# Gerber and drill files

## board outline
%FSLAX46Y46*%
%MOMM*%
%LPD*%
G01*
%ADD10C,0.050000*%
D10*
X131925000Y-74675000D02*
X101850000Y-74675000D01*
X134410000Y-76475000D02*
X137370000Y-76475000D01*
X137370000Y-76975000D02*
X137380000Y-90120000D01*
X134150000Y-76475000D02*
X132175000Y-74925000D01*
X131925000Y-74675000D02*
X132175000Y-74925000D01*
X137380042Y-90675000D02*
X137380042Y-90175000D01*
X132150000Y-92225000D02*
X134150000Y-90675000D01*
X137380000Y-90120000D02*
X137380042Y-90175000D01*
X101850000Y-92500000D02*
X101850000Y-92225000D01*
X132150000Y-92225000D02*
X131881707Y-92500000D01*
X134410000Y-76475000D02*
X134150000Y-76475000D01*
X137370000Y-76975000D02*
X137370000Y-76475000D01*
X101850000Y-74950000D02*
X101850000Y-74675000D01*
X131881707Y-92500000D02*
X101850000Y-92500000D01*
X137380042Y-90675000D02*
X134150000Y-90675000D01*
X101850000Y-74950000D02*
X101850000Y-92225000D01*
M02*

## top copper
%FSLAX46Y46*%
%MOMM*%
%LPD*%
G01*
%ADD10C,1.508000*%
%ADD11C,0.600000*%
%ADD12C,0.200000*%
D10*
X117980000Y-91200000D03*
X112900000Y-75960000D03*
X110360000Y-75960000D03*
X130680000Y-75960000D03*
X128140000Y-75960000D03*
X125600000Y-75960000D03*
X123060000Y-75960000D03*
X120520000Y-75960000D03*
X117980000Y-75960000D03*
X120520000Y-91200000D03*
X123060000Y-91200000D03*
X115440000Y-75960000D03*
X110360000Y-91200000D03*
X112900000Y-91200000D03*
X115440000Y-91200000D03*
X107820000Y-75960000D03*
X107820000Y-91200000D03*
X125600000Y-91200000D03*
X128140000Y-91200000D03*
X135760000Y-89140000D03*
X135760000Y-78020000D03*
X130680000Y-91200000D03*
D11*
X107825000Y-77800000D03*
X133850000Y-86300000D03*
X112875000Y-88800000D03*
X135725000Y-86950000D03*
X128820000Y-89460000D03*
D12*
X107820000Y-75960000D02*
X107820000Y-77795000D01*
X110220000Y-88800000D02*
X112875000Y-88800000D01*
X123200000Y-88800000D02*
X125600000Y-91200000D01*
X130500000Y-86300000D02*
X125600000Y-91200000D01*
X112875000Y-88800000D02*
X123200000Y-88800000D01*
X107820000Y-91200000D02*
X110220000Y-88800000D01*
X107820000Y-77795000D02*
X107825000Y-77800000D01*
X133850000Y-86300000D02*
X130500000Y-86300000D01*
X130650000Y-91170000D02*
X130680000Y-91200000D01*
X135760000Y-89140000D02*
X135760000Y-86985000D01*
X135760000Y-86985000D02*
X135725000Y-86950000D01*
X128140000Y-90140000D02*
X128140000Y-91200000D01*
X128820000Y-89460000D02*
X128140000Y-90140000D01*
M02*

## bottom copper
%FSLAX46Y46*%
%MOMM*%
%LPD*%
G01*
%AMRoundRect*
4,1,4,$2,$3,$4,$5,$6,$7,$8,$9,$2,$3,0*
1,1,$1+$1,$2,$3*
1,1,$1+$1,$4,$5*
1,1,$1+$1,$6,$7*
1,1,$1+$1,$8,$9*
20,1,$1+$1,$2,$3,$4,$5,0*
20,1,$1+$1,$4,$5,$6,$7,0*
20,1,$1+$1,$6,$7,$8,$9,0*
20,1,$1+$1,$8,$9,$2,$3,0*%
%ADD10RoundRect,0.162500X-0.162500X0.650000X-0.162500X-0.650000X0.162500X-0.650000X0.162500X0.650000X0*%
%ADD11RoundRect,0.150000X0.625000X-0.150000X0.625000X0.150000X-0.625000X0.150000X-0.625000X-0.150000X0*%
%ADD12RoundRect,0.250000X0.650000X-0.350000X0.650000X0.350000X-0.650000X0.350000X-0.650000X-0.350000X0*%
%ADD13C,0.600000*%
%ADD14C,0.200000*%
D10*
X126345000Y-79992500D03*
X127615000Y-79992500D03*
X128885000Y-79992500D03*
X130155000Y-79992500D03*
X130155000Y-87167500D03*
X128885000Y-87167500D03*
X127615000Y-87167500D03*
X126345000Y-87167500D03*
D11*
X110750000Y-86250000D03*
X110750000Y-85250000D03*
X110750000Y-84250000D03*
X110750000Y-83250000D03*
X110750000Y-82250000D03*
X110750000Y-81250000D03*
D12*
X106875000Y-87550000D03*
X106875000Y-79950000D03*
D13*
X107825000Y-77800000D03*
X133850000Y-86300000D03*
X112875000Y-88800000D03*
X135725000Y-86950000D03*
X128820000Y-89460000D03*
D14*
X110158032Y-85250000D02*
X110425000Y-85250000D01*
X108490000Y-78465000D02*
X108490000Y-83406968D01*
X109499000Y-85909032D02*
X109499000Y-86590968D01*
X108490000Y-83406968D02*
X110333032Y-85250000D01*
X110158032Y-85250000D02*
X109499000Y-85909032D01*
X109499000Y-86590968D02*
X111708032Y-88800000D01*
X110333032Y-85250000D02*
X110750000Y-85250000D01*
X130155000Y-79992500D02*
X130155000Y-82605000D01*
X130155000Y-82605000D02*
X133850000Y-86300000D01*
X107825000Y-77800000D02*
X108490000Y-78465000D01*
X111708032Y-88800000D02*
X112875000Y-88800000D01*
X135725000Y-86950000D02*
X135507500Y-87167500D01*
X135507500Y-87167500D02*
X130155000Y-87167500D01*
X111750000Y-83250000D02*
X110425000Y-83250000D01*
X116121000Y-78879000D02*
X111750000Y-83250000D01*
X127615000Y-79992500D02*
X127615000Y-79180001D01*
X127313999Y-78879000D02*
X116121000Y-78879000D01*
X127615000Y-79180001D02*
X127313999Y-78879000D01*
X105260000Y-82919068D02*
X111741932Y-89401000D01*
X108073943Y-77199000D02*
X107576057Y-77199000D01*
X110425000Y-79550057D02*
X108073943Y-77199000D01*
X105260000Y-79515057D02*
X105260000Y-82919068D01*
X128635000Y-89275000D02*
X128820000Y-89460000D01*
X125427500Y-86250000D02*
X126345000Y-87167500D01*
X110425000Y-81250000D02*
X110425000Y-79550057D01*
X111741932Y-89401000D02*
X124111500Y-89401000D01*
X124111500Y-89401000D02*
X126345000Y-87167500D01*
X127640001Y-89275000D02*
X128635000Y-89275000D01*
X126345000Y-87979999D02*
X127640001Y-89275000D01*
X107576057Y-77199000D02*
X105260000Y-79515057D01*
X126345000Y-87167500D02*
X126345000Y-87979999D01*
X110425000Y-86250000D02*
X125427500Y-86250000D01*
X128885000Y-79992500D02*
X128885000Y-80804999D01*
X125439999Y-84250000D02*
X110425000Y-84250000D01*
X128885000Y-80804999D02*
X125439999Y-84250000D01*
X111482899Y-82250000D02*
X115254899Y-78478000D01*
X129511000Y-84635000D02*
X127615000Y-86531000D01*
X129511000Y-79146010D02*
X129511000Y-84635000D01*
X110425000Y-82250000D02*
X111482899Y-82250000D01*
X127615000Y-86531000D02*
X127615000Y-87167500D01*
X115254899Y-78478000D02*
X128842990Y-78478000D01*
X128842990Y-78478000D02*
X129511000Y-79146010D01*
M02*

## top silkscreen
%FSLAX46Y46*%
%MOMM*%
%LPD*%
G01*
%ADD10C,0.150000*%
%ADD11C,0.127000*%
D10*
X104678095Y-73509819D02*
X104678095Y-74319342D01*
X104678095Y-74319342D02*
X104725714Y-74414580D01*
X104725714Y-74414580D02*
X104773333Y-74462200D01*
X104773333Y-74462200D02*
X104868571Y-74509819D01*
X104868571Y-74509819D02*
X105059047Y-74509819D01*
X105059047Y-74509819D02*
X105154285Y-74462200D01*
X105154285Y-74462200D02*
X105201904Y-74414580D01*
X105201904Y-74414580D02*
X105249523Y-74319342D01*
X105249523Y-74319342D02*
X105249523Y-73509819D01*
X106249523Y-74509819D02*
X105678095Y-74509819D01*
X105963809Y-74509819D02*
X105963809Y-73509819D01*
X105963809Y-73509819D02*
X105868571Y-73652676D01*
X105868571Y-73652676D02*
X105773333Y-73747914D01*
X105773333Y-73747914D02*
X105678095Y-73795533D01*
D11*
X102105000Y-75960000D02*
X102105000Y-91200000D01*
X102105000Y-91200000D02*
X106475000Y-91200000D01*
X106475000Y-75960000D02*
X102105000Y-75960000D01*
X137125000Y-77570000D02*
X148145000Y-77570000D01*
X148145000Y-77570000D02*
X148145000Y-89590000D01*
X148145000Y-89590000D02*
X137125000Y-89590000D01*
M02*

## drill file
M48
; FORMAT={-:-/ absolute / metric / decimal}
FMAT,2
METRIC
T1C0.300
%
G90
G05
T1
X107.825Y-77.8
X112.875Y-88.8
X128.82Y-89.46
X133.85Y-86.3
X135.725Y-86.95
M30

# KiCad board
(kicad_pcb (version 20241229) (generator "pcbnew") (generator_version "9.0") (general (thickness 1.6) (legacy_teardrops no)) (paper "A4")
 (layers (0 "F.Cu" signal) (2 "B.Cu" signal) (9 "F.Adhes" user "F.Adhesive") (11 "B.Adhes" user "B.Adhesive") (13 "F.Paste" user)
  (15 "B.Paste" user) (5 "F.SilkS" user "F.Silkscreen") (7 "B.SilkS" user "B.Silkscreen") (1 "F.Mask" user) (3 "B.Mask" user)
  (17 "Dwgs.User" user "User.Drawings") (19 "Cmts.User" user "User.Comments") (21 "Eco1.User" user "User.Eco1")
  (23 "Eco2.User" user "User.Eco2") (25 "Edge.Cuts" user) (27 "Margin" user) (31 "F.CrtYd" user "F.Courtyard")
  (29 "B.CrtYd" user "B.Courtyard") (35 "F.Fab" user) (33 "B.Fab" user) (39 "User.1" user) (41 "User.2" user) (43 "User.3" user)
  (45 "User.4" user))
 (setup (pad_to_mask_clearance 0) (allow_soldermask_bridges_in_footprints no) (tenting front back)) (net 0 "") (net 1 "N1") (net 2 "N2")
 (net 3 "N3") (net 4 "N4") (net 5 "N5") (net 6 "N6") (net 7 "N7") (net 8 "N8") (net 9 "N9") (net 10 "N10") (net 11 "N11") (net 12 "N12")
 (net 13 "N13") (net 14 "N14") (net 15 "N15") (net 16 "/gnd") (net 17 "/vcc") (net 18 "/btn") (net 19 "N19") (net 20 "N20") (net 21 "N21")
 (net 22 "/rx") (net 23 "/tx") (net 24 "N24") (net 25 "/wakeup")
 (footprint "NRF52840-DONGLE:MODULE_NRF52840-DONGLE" (layer "F.Cu") (at 125.125 83.58)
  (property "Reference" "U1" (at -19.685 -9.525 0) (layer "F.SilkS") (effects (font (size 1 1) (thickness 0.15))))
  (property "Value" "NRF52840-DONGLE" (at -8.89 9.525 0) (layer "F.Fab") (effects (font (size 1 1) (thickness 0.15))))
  (fp_line (start -23.02 -7.62) (end -23.02 7.62) (stroke (width 0.127) (type solid)) (layer "F.SilkS"))
  (fp_line (start -23.02 7.62) (end -18.65 7.62) (stroke (width 0.127) (type solid)) (layer "F.SilkS"))
  (fp_line (start -18.65 -7.62) (end -23.02 -7.62) (stroke (width 0.127) (type solid)) (layer "F.SilkS"))
  (fp_line (start 12 -6.01) (end 23.02 -6.01) (stroke (width 0.127) (type solid)) (layer "F.SilkS"))
  (fp_line (start 23.02 -6.01) (end 23.02 6.01) (stroke (width 0.127) (type solid)) (layer "F.SilkS"))
  (fp_line (start 23.02 6.01) (end 12 6.01) (stroke (width 0.127) (type solid)) (layer "F.SilkS"))
  (pad "0.02" smd circle (at -7.145 7.62) (size 1.508 1.508) (layers "F.Cu") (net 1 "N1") (solder_mask_margin 0.102))
  (pad "0.09" smd circle (at -12.225 -7.62) (size 1.508 1.508) (layers "F.Cu") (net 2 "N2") (solder_mask_margin 0.102))
  (pad "0.10" smd circle (at -14.765 -7.62) (size 1.508 1.508) (layers "F.Cu") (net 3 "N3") (solder_mask_margin 0.102))
  (pad "0.13" smd circle (at 5.555 -7.62) (size 1.508 1.508) (layers "F.Cu") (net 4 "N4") (solder_mask_margin 0.102))
  (pad "0.15" smd circle (at 3.015 -7.62) (size 1.508 1.508) (layers "F.Cu") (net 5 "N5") (solder_mask_margin 0.102))
  (pad "0.17" smd circle (at 0.475 -7.62) (size 1.508 1.508) (layers "F.Cu") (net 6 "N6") (solder_mask_margin 0.102))
  (pad "0.20" smd circle (at -2.065 -7.62) (size 1.508 1.508) (layers "F.Cu") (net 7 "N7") (solder_mask_margin 0.102))
  (pad "0.22" smd circle (at -4.605 -7.62) (size 1.508 1.508) (layers "F.Cu") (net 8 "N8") (solder_mask_margin 0.102))
  (pad "0.24" smd circle (at -7.145 -7.62) (size 1.508 1.508) (layers "F.Cu") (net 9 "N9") (solder_mask_margin 0.102))
  (pad "0.29" smd circle (at -4.605 7.62) (size 1.508 1.508) (layers "F.Cu") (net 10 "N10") (solder_mask_margin 0.102))
  (pad "0.31" smd circle (at -2.065 7.62) (size 1.508 1.508) (layers "F.Cu") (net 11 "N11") (solder_mask_margin 0.102))
  (pad "1.00" smd circle (at -9.685 -7.62) (size 1.508 1.508) (layers "F.Cu") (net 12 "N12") (solder_mask_margin 0.102))
  (pad "1.10" smd circle (at -14.765 7.62) (size 1.508 1.508) (layers "F.Cu") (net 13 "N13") (solder_mask_margin 0.102))
  (pad "1.13" smd circle (at -12.225 7.62) (size 1.508 1.508) (layers "F.Cu") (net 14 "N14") (solder_mask_margin 0.102))
  (pad "1.15" smd circle (at -9.685 7.62) (size 1.508 1.508) (layers "F.Cu") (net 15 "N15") (solder_mask_margin 0.102))
  (pad "G1" smd circle (at -17.305 -7.62) (size 1.508 1.508) (layers "F.Cu") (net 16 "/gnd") (solder_mask_margin 0.102)
   (padstack (mode front_inner_back)
    (layer "Inner" (shape circle) (size 1.508 1.508) (zone_connect -1))
    (layer "B.Cu" (shape circle) (size 1.508 1.508) (zone_connect -1))))
  (pad "G2" smd circle (at -17.305 7.62) (size 1.508 1.508) (layers "F.Cu") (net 16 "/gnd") (solder_mask_margin 0.102))
  (pad "G3" smd circle (at 0.475 7.62) (size 1.508 1.508) (layers "F.Cu") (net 16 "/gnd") (solder_mask_margin 0.102))
  (pad "OUT" smd circle (at 3.015 7.62) (size 1.508 1.508) (layers "F.Cu") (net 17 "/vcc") (solder_mask_margin 0.102))
  (pad "SWDCLK" smd circle (at 10.635 5.56) (size 1.508 1.508) (layers "F.Cu") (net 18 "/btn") (solder_mask_margin 0.102))
  (pad "SWDIO" smd circle (at 10.635 -5.56) (size 1.508 1.508) (layers "F.Cu") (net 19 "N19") (solder_mask_margin 0.102))
  (pad "VBUS" smd circle (at 5.555 7.62) (size 1.508 1.508) (layers "F.Cu") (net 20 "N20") (solder_mask_margin 0.102)))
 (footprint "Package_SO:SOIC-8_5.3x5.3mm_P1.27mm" (layer "B.Cu") (at 128.25 83.58 -90)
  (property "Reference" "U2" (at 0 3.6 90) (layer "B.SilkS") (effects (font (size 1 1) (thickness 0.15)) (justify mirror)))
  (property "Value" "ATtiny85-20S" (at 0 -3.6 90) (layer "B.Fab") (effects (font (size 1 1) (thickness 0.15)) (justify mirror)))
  (pad "1" smd roundrect (at -3.5875 1.905 270) (size 1.625 0.65) (layers "B.Cu" "B.Mask" "B.Paste") (roundrect_rratio 0.25) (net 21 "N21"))
  (pad "2" smd roundrect (at -3.5875 0.635 270) (size 1.625 0.65) (layers "B.Cu" "B.Mask" "B.Paste") (roundrect_rratio 0.25) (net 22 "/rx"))
  (pad "3" smd roundrect (at -3.5875 -0.635 270) (size 1.625 0.65) (layers "B.Cu" "B.Mask" "B.Paste") (roundrect_rratio 0.25) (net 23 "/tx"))
  (pad "4" smd roundrect (at -3.5875 -1.905 270) (size 1.625 0.65) (layers "B.Cu" "B.Mask" "B.Paste") (roundrect_rratio 0.25)
   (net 16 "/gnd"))
  (pad "5" smd roundrect (at 3.5875 -1.905 270) (size 1.625 0.65) (layers "B.Cu" "B.Mask" "B.Paste") (roundrect_rratio 0.25) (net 18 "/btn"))
  (pad "6" smd roundrect (at 3.5875 -0.635 270) (size 1.625 0.65) (layers "B.Cu" "B.Mask" "B.Paste") (roundrect_rratio 0.25) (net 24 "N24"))
  (pad "7" smd roundrect (at 3.5875 0.635 270) (size 1.625 0.65) (layers "B.Cu" "B.Mask" "B.Paste") (roundrect_rratio 0.25)
   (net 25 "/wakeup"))
  (pad "8" smd roundrect (at 3.5875 1.905 270) (size 1.625 0.65) (layers "B.Cu" "B.Mask" "B.Paste") (roundrect_rratio 0.25) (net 17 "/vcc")))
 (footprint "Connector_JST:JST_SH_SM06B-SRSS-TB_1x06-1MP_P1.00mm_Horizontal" (layer "B.Cu") (at 108.75 83.75 90)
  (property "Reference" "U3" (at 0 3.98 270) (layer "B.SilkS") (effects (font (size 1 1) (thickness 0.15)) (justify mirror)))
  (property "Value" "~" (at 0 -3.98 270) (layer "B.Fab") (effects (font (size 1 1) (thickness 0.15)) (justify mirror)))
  (pad "1" smd roundrect (at -2.5 2 90) (size 0.6 1.55) (layers "B.Cu" "B.Mask" "B.Paste") (roundrect_rratio 0.25) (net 17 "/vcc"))
  (pad "2" smd roundrect (at -1.5 2 90) (size 0.6 1.55) (layers "B.Cu" "B.Mask" "B.Paste") (roundrect_rratio 0.25) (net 16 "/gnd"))
  (pad "3" smd roundrect (at -0.5 2 90) (size 0.6 1.55) (layers "B.Cu" "B.Mask" "B.Paste") (roundrect_rratio 0.25) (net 23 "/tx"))
  (pad "4" smd roundrect (at 0.5 2 90) (size 0.6 1.55) (layers "B.Cu" "B.Mask" "B.Paste") (roundrect_rratio 0.25) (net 22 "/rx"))
  (pad "5" smd roundrect (at 1.5 2 90) (size 0.6 1.55) (layers "B.Cu" "B.Mask" "B.Paste") (roundrect_rratio 0.25) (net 25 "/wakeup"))
  (pad "6" smd roundrect (at 2.5 2 90) (size 0.6 1.55) (layers "B.Cu" "B.Mask" "B.Paste") (roundrect_rratio 0.25) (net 17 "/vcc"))
  (pad "MP" smd roundrect (at -3.8 -1.875 90) (size 1.2 1.8) (layers "B.Cu" "B.Mask" "B.Paste") (roundrect_rratio 0.208333))
  (pad "MP" smd roundrect (at 3.8 -1.875 90) (size 1.2 1.8) (layers "B.Cu" "B.Mask" "B.Paste") (roundrect_rratio 0.208333)))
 (gr_line (start 131.925 74.675) (end 101.85 74.675) (stroke (width 0.05) (type default)) (layer "Edge.Cuts"))
 (gr_line (start 134.41 76.475) (end 137.37 76.475) (stroke (width 0.05) (type solid)) (layer "Edge.Cuts"))
 (gr_line (start 137.37 76.975) (end 137.38 90.12) (stroke (width 0.05) (type default)) (layer "Edge.Cuts"))
 (gr_line (start 134.15 76.475) (end 132.175 74.925) (stroke (width 0.05) (type default)) (layer "Edge.Cuts"))
 (gr_line (start 131.925 74.675) (end 132.175 74.925) (stroke (width 0.05) (type default)) (layer "Edge.Cuts"))
 (gr_line (start 137.380042 90.675) (end 137.380042 90.175) (stroke (width 0.05) (type default)) (layer "Edge.Cuts"))
 (gr_line (start 132.15 92.225) (end 134.15 90.675) (stroke (width 0.05) (type default)) (layer "Edge.Cuts"))
 (gr_line (start 137.38 90.12) (end 137.380042 90.175) (stroke (width 0.05) (type default)) (layer "Edge.Cuts"))
 (gr_line (start 101.85 92.5) (end 101.85 92.225) (stroke (width 0.05) (type default)) (layer "Edge.Cuts"))
 (gr_line (start 132.15 92.225) (end 131.881707 92.5) (stroke (width 0.05) (type default)) (layer "Edge.Cuts"))
 (gr_line (start 134.41 76.475) (end 134.15 76.475) (stroke (width 0.05) (type solid)) (layer "Edge.Cuts"))
 (gr_line (start 137.37 76.975) (end 137.37 76.475) (stroke (width 0.05) (type default)) (layer "Edge.Cuts"))
 (gr_line (start 101.85 74.95) (end 101.85 74.675) (stroke (width 0.05) (type default)) (layer "Edge.Cuts"))
 (gr_line (start 131.881707 92.5) (end 101.85 92.5) (stroke (width 0.05) (type default)) (layer "Edge.Cuts"))
 (gr_line (start 137.380042 90.675) (end 134.15 90.675) (stroke (width 0.05) (type solid)) (layer "Edge.Cuts"))
 (gr_line (start 101.85 74.95) (end 101.85 92.225) (stroke (width 0.05) (type default)) (layer "Edge.Cuts"))
 (segment (start 107.82 75.96) (end 107.82 77.795) (width 0.2) (layer "F.Cu") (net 16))
 (segment (start 110.22 88.8) (end 112.875 88.8) (width 0.2) (layer "F.Cu") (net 16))
 (segment (start 123.2 88.8) (end 125.6 91.2) (width 0.2) (layer "F.Cu") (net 16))
 (segment (start 130.5 86.3) (end 125.6 91.2) (width 0.2) (layer "F.Cu") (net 16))
 (segment (start 112.875 88.8) (end 123.2 88.8) (width 0.2) (layer "F.Cu") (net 16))
 (segment (start 107.82 91.2) (end 110.22 88.8) (width 0.2) (layer "F.Cu") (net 16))
 (segment (start 107.82 77.795) (end 107.825 77.8) (width 0.2) (layer "F.Cu") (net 16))
 (segment (start 133.85 86.3) (end 130.5 86.3) (width 0.2) (layer "F.Cu") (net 16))
 (via (at 107.825 77.8) (size 0.6) (drill 0.3) (layers "F.Cu" "B.Cu") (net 16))
 (via (at 133.85 86.3) (size 0.6) (drill 0.3) (layers "F.Cu" "B.Cu") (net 16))
 (via (at 112.875 88.8) (size 0.6) (drill 0.3) (layers "F.Cu" "B.Cu") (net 16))
 (segment (start 110.158032 85.25) (end 110.425 85.25) (width 0.2) (layer "B.Cu") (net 16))
 (segment (start 108.49 78.465) (end 108.49 83.406968) (width 0.2) (layer "B.Cu") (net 16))
 (segment (start 109.499 85.909032) (end 109.499 86.590968) (width 0.2) (layer "B.Cu") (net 16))
 (segment (start 108.49 83.406968) (end 110.333032 85.25) (width 0.2) (layer "B.Cu") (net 16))
 (segment (start 110.158032 85.25) (end 109.499 85.909032) (width 0.2) (layer "B.Cu") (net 16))
 (segment (start 109.499 86.590968) (end 111.708032 88.8) (width 0.2) (layer "B.Cu") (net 16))
 (segment (start 110.333032 85.25) (end 110.75 85.25) (width 0.2) (layer "B.Cu") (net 16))
 (segment (start 130.155 79.9925) (end 130.155 82.605) (width 0.2) (layer "B.Cu") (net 16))
 (segment (start 130.155 82.605) (end 133.85 86.3) (width 0.2) (layer "B.Cu") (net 16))
 (segment (start 107.825 77.8) (end 108.49 78.465) (width 0.2) (layer "B.Cu") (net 16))
 (segment (start 111.708032 88.8) (end 112.875 88.8) (width 0.2) (layer "B.Cu") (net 16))
 (segment (start 130.65 91.17) (end 130.68 91.2) (width 0.2) (layer "F.Cu") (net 20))
 (segment (start 135.76 89.14) (end 135.76 86.985) (width 0.2) (layer "F.Cu") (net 18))
 (segment (start 135.76 86.985) (end 135.725 86.95) (width 0.2) (layer "F.Cu") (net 18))
 (via (at 135.725 86.95) (size 0.6) (drill 0.3) (layers "F.Cu" "B.Cu") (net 18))
 (segment (start 135.725 86.95) (end 135.5075 87.1675) (width 0.2) (layer "B.Cu") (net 18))
 (segment (start 135.5075 87.1675) (end 130.155 87.1675) (width 0.2) (layer "B.Cu") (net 18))
 (segment (start 111.75 83.25) (end 110.425 83.25) (width 0.2) (layer "B.Cu") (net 22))
 (segment (start 116.121 78.879) (end 111.75 83.25) (width 0.2) (layer "B.Cu") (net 22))
 (segment (start 127.615 79.9925) (end 127.615 79.180001) (width 0.2) (layer "B.Cu") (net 22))
 (segment (start 127.313999 78.879) (end 116.121 78.879) (width 0.2) (layer "B.Cu") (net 22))
 (segment (start 127.615 79.180001) (end 127.313999 78.879) (width 0.2) (layer "B.Cu") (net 22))
 (segment (start 128.14 90.14) (end 128.14 91.2) (width 0.2) (layer "F.Cu") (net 17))
 (segment (start 128.82 89.46) (end 128.14 90.14) (width 0.2) (layer "F.Cu") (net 17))
 (via (at 128.82 89.46) (size 0.6) (drill 0.3) (layers "F.Cu" "B.Cu") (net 17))
 (segment (start 105.26 82.919068) (end 111.741932 89.401) (width 0.2) (layer "B.Cu") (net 17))
 (segment (start 108.073943 77.199) (end 107.576057 77.199) (width 0.2) (layer "B.Cu") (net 17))
 (segment (start 110.425 79.550057) (end 108.073943 77.199) (width 0.2) (layer "B.Cu") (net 17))
 (segment (start 105.26 79.515057) (end 105.26 82.919068) (width 0.2) (layer "B.Cu") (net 17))
 (segment (start 128.635 89.275) (end 128.82 89.46) (width 0.2) (layer "B.Cu") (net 17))
 (segment (start 125.4275 86.25) (end 126.345 87.1675) (width 0.2) (layer "B.Cu") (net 17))
 (segment (start 110.425 81.25) (end 110.425 79.550057) (width 0.2) (layer "B.Cu") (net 17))
 (segment (start 111.741932 89.401) (end 124.1115 89.401) (width 0.2) (layer "B.Cu") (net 17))
 (segment (start 124.1115 89.401) (end 126.345 87.1675) (width 0.2) (layer "B.Cu") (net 17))
 (segment (start 127.640001 89.275) (end 128.635 89.275) (width 0.2) (layer "B.Cu") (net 17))
 (segment (start 126.345 87.979999) (end 127.640001 89.275) (width 0.2) (layer "B.Cu") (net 17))
 (segment (start 107.576057 77.199) (end 105.26 79.515057) (width 0.2) (layer "B.Cu") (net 17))
 (segment (start 126.345 87.1675) (end 126.345 87.979999) (width 0.2) (layer "B.Cu") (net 17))
 (segment (start 110.425 86.25) (end 125.4275 86.25) (width 0.2) (layer "B.Cu") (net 17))
 (segment (start 128.885 79.9925) (end 128.885 80.804999) (width 0.2) (layer "B.Cu") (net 23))
 (segment (start 125.439999 84.25) (end 110.425 84.25) (width 0.2) (layer "B.Cu") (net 23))
 (segment (start 128.885 80.804999) (end 125.439999 84.25) (width 0.2) (layer "B.Cu") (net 23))
 (segment (start 111.482899 82.25) (end 115.254899 78.478) (width 0.2) (layer "B.Cu") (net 25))
 (segment (start 129.511 84.635) (end 127.615 86.531) (width 0.2) (layer "B.Cu") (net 25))
 (segment (start 129.511 79.14601) (end 129.511 84.635) (width 0.2) (layer "B.Cu") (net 25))
 (segment (start 110.425 82.25) (end 111.482899 82.25) (width 0.2) (layer "B.Cu") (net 25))
 (segment (start 127.615 86.531) (end 127.615 87.1675) (width 0.2) (layer "B.Cu") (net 25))
 (segment (start 115.254899 78.478) (end 128.84299 78.478) (width 0.2) (layer "B.Cu") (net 25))
 (segment (start 128.84299 78.478) (end 129.511 79.14601) (width 0.2) (layer "B.Cu") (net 25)))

